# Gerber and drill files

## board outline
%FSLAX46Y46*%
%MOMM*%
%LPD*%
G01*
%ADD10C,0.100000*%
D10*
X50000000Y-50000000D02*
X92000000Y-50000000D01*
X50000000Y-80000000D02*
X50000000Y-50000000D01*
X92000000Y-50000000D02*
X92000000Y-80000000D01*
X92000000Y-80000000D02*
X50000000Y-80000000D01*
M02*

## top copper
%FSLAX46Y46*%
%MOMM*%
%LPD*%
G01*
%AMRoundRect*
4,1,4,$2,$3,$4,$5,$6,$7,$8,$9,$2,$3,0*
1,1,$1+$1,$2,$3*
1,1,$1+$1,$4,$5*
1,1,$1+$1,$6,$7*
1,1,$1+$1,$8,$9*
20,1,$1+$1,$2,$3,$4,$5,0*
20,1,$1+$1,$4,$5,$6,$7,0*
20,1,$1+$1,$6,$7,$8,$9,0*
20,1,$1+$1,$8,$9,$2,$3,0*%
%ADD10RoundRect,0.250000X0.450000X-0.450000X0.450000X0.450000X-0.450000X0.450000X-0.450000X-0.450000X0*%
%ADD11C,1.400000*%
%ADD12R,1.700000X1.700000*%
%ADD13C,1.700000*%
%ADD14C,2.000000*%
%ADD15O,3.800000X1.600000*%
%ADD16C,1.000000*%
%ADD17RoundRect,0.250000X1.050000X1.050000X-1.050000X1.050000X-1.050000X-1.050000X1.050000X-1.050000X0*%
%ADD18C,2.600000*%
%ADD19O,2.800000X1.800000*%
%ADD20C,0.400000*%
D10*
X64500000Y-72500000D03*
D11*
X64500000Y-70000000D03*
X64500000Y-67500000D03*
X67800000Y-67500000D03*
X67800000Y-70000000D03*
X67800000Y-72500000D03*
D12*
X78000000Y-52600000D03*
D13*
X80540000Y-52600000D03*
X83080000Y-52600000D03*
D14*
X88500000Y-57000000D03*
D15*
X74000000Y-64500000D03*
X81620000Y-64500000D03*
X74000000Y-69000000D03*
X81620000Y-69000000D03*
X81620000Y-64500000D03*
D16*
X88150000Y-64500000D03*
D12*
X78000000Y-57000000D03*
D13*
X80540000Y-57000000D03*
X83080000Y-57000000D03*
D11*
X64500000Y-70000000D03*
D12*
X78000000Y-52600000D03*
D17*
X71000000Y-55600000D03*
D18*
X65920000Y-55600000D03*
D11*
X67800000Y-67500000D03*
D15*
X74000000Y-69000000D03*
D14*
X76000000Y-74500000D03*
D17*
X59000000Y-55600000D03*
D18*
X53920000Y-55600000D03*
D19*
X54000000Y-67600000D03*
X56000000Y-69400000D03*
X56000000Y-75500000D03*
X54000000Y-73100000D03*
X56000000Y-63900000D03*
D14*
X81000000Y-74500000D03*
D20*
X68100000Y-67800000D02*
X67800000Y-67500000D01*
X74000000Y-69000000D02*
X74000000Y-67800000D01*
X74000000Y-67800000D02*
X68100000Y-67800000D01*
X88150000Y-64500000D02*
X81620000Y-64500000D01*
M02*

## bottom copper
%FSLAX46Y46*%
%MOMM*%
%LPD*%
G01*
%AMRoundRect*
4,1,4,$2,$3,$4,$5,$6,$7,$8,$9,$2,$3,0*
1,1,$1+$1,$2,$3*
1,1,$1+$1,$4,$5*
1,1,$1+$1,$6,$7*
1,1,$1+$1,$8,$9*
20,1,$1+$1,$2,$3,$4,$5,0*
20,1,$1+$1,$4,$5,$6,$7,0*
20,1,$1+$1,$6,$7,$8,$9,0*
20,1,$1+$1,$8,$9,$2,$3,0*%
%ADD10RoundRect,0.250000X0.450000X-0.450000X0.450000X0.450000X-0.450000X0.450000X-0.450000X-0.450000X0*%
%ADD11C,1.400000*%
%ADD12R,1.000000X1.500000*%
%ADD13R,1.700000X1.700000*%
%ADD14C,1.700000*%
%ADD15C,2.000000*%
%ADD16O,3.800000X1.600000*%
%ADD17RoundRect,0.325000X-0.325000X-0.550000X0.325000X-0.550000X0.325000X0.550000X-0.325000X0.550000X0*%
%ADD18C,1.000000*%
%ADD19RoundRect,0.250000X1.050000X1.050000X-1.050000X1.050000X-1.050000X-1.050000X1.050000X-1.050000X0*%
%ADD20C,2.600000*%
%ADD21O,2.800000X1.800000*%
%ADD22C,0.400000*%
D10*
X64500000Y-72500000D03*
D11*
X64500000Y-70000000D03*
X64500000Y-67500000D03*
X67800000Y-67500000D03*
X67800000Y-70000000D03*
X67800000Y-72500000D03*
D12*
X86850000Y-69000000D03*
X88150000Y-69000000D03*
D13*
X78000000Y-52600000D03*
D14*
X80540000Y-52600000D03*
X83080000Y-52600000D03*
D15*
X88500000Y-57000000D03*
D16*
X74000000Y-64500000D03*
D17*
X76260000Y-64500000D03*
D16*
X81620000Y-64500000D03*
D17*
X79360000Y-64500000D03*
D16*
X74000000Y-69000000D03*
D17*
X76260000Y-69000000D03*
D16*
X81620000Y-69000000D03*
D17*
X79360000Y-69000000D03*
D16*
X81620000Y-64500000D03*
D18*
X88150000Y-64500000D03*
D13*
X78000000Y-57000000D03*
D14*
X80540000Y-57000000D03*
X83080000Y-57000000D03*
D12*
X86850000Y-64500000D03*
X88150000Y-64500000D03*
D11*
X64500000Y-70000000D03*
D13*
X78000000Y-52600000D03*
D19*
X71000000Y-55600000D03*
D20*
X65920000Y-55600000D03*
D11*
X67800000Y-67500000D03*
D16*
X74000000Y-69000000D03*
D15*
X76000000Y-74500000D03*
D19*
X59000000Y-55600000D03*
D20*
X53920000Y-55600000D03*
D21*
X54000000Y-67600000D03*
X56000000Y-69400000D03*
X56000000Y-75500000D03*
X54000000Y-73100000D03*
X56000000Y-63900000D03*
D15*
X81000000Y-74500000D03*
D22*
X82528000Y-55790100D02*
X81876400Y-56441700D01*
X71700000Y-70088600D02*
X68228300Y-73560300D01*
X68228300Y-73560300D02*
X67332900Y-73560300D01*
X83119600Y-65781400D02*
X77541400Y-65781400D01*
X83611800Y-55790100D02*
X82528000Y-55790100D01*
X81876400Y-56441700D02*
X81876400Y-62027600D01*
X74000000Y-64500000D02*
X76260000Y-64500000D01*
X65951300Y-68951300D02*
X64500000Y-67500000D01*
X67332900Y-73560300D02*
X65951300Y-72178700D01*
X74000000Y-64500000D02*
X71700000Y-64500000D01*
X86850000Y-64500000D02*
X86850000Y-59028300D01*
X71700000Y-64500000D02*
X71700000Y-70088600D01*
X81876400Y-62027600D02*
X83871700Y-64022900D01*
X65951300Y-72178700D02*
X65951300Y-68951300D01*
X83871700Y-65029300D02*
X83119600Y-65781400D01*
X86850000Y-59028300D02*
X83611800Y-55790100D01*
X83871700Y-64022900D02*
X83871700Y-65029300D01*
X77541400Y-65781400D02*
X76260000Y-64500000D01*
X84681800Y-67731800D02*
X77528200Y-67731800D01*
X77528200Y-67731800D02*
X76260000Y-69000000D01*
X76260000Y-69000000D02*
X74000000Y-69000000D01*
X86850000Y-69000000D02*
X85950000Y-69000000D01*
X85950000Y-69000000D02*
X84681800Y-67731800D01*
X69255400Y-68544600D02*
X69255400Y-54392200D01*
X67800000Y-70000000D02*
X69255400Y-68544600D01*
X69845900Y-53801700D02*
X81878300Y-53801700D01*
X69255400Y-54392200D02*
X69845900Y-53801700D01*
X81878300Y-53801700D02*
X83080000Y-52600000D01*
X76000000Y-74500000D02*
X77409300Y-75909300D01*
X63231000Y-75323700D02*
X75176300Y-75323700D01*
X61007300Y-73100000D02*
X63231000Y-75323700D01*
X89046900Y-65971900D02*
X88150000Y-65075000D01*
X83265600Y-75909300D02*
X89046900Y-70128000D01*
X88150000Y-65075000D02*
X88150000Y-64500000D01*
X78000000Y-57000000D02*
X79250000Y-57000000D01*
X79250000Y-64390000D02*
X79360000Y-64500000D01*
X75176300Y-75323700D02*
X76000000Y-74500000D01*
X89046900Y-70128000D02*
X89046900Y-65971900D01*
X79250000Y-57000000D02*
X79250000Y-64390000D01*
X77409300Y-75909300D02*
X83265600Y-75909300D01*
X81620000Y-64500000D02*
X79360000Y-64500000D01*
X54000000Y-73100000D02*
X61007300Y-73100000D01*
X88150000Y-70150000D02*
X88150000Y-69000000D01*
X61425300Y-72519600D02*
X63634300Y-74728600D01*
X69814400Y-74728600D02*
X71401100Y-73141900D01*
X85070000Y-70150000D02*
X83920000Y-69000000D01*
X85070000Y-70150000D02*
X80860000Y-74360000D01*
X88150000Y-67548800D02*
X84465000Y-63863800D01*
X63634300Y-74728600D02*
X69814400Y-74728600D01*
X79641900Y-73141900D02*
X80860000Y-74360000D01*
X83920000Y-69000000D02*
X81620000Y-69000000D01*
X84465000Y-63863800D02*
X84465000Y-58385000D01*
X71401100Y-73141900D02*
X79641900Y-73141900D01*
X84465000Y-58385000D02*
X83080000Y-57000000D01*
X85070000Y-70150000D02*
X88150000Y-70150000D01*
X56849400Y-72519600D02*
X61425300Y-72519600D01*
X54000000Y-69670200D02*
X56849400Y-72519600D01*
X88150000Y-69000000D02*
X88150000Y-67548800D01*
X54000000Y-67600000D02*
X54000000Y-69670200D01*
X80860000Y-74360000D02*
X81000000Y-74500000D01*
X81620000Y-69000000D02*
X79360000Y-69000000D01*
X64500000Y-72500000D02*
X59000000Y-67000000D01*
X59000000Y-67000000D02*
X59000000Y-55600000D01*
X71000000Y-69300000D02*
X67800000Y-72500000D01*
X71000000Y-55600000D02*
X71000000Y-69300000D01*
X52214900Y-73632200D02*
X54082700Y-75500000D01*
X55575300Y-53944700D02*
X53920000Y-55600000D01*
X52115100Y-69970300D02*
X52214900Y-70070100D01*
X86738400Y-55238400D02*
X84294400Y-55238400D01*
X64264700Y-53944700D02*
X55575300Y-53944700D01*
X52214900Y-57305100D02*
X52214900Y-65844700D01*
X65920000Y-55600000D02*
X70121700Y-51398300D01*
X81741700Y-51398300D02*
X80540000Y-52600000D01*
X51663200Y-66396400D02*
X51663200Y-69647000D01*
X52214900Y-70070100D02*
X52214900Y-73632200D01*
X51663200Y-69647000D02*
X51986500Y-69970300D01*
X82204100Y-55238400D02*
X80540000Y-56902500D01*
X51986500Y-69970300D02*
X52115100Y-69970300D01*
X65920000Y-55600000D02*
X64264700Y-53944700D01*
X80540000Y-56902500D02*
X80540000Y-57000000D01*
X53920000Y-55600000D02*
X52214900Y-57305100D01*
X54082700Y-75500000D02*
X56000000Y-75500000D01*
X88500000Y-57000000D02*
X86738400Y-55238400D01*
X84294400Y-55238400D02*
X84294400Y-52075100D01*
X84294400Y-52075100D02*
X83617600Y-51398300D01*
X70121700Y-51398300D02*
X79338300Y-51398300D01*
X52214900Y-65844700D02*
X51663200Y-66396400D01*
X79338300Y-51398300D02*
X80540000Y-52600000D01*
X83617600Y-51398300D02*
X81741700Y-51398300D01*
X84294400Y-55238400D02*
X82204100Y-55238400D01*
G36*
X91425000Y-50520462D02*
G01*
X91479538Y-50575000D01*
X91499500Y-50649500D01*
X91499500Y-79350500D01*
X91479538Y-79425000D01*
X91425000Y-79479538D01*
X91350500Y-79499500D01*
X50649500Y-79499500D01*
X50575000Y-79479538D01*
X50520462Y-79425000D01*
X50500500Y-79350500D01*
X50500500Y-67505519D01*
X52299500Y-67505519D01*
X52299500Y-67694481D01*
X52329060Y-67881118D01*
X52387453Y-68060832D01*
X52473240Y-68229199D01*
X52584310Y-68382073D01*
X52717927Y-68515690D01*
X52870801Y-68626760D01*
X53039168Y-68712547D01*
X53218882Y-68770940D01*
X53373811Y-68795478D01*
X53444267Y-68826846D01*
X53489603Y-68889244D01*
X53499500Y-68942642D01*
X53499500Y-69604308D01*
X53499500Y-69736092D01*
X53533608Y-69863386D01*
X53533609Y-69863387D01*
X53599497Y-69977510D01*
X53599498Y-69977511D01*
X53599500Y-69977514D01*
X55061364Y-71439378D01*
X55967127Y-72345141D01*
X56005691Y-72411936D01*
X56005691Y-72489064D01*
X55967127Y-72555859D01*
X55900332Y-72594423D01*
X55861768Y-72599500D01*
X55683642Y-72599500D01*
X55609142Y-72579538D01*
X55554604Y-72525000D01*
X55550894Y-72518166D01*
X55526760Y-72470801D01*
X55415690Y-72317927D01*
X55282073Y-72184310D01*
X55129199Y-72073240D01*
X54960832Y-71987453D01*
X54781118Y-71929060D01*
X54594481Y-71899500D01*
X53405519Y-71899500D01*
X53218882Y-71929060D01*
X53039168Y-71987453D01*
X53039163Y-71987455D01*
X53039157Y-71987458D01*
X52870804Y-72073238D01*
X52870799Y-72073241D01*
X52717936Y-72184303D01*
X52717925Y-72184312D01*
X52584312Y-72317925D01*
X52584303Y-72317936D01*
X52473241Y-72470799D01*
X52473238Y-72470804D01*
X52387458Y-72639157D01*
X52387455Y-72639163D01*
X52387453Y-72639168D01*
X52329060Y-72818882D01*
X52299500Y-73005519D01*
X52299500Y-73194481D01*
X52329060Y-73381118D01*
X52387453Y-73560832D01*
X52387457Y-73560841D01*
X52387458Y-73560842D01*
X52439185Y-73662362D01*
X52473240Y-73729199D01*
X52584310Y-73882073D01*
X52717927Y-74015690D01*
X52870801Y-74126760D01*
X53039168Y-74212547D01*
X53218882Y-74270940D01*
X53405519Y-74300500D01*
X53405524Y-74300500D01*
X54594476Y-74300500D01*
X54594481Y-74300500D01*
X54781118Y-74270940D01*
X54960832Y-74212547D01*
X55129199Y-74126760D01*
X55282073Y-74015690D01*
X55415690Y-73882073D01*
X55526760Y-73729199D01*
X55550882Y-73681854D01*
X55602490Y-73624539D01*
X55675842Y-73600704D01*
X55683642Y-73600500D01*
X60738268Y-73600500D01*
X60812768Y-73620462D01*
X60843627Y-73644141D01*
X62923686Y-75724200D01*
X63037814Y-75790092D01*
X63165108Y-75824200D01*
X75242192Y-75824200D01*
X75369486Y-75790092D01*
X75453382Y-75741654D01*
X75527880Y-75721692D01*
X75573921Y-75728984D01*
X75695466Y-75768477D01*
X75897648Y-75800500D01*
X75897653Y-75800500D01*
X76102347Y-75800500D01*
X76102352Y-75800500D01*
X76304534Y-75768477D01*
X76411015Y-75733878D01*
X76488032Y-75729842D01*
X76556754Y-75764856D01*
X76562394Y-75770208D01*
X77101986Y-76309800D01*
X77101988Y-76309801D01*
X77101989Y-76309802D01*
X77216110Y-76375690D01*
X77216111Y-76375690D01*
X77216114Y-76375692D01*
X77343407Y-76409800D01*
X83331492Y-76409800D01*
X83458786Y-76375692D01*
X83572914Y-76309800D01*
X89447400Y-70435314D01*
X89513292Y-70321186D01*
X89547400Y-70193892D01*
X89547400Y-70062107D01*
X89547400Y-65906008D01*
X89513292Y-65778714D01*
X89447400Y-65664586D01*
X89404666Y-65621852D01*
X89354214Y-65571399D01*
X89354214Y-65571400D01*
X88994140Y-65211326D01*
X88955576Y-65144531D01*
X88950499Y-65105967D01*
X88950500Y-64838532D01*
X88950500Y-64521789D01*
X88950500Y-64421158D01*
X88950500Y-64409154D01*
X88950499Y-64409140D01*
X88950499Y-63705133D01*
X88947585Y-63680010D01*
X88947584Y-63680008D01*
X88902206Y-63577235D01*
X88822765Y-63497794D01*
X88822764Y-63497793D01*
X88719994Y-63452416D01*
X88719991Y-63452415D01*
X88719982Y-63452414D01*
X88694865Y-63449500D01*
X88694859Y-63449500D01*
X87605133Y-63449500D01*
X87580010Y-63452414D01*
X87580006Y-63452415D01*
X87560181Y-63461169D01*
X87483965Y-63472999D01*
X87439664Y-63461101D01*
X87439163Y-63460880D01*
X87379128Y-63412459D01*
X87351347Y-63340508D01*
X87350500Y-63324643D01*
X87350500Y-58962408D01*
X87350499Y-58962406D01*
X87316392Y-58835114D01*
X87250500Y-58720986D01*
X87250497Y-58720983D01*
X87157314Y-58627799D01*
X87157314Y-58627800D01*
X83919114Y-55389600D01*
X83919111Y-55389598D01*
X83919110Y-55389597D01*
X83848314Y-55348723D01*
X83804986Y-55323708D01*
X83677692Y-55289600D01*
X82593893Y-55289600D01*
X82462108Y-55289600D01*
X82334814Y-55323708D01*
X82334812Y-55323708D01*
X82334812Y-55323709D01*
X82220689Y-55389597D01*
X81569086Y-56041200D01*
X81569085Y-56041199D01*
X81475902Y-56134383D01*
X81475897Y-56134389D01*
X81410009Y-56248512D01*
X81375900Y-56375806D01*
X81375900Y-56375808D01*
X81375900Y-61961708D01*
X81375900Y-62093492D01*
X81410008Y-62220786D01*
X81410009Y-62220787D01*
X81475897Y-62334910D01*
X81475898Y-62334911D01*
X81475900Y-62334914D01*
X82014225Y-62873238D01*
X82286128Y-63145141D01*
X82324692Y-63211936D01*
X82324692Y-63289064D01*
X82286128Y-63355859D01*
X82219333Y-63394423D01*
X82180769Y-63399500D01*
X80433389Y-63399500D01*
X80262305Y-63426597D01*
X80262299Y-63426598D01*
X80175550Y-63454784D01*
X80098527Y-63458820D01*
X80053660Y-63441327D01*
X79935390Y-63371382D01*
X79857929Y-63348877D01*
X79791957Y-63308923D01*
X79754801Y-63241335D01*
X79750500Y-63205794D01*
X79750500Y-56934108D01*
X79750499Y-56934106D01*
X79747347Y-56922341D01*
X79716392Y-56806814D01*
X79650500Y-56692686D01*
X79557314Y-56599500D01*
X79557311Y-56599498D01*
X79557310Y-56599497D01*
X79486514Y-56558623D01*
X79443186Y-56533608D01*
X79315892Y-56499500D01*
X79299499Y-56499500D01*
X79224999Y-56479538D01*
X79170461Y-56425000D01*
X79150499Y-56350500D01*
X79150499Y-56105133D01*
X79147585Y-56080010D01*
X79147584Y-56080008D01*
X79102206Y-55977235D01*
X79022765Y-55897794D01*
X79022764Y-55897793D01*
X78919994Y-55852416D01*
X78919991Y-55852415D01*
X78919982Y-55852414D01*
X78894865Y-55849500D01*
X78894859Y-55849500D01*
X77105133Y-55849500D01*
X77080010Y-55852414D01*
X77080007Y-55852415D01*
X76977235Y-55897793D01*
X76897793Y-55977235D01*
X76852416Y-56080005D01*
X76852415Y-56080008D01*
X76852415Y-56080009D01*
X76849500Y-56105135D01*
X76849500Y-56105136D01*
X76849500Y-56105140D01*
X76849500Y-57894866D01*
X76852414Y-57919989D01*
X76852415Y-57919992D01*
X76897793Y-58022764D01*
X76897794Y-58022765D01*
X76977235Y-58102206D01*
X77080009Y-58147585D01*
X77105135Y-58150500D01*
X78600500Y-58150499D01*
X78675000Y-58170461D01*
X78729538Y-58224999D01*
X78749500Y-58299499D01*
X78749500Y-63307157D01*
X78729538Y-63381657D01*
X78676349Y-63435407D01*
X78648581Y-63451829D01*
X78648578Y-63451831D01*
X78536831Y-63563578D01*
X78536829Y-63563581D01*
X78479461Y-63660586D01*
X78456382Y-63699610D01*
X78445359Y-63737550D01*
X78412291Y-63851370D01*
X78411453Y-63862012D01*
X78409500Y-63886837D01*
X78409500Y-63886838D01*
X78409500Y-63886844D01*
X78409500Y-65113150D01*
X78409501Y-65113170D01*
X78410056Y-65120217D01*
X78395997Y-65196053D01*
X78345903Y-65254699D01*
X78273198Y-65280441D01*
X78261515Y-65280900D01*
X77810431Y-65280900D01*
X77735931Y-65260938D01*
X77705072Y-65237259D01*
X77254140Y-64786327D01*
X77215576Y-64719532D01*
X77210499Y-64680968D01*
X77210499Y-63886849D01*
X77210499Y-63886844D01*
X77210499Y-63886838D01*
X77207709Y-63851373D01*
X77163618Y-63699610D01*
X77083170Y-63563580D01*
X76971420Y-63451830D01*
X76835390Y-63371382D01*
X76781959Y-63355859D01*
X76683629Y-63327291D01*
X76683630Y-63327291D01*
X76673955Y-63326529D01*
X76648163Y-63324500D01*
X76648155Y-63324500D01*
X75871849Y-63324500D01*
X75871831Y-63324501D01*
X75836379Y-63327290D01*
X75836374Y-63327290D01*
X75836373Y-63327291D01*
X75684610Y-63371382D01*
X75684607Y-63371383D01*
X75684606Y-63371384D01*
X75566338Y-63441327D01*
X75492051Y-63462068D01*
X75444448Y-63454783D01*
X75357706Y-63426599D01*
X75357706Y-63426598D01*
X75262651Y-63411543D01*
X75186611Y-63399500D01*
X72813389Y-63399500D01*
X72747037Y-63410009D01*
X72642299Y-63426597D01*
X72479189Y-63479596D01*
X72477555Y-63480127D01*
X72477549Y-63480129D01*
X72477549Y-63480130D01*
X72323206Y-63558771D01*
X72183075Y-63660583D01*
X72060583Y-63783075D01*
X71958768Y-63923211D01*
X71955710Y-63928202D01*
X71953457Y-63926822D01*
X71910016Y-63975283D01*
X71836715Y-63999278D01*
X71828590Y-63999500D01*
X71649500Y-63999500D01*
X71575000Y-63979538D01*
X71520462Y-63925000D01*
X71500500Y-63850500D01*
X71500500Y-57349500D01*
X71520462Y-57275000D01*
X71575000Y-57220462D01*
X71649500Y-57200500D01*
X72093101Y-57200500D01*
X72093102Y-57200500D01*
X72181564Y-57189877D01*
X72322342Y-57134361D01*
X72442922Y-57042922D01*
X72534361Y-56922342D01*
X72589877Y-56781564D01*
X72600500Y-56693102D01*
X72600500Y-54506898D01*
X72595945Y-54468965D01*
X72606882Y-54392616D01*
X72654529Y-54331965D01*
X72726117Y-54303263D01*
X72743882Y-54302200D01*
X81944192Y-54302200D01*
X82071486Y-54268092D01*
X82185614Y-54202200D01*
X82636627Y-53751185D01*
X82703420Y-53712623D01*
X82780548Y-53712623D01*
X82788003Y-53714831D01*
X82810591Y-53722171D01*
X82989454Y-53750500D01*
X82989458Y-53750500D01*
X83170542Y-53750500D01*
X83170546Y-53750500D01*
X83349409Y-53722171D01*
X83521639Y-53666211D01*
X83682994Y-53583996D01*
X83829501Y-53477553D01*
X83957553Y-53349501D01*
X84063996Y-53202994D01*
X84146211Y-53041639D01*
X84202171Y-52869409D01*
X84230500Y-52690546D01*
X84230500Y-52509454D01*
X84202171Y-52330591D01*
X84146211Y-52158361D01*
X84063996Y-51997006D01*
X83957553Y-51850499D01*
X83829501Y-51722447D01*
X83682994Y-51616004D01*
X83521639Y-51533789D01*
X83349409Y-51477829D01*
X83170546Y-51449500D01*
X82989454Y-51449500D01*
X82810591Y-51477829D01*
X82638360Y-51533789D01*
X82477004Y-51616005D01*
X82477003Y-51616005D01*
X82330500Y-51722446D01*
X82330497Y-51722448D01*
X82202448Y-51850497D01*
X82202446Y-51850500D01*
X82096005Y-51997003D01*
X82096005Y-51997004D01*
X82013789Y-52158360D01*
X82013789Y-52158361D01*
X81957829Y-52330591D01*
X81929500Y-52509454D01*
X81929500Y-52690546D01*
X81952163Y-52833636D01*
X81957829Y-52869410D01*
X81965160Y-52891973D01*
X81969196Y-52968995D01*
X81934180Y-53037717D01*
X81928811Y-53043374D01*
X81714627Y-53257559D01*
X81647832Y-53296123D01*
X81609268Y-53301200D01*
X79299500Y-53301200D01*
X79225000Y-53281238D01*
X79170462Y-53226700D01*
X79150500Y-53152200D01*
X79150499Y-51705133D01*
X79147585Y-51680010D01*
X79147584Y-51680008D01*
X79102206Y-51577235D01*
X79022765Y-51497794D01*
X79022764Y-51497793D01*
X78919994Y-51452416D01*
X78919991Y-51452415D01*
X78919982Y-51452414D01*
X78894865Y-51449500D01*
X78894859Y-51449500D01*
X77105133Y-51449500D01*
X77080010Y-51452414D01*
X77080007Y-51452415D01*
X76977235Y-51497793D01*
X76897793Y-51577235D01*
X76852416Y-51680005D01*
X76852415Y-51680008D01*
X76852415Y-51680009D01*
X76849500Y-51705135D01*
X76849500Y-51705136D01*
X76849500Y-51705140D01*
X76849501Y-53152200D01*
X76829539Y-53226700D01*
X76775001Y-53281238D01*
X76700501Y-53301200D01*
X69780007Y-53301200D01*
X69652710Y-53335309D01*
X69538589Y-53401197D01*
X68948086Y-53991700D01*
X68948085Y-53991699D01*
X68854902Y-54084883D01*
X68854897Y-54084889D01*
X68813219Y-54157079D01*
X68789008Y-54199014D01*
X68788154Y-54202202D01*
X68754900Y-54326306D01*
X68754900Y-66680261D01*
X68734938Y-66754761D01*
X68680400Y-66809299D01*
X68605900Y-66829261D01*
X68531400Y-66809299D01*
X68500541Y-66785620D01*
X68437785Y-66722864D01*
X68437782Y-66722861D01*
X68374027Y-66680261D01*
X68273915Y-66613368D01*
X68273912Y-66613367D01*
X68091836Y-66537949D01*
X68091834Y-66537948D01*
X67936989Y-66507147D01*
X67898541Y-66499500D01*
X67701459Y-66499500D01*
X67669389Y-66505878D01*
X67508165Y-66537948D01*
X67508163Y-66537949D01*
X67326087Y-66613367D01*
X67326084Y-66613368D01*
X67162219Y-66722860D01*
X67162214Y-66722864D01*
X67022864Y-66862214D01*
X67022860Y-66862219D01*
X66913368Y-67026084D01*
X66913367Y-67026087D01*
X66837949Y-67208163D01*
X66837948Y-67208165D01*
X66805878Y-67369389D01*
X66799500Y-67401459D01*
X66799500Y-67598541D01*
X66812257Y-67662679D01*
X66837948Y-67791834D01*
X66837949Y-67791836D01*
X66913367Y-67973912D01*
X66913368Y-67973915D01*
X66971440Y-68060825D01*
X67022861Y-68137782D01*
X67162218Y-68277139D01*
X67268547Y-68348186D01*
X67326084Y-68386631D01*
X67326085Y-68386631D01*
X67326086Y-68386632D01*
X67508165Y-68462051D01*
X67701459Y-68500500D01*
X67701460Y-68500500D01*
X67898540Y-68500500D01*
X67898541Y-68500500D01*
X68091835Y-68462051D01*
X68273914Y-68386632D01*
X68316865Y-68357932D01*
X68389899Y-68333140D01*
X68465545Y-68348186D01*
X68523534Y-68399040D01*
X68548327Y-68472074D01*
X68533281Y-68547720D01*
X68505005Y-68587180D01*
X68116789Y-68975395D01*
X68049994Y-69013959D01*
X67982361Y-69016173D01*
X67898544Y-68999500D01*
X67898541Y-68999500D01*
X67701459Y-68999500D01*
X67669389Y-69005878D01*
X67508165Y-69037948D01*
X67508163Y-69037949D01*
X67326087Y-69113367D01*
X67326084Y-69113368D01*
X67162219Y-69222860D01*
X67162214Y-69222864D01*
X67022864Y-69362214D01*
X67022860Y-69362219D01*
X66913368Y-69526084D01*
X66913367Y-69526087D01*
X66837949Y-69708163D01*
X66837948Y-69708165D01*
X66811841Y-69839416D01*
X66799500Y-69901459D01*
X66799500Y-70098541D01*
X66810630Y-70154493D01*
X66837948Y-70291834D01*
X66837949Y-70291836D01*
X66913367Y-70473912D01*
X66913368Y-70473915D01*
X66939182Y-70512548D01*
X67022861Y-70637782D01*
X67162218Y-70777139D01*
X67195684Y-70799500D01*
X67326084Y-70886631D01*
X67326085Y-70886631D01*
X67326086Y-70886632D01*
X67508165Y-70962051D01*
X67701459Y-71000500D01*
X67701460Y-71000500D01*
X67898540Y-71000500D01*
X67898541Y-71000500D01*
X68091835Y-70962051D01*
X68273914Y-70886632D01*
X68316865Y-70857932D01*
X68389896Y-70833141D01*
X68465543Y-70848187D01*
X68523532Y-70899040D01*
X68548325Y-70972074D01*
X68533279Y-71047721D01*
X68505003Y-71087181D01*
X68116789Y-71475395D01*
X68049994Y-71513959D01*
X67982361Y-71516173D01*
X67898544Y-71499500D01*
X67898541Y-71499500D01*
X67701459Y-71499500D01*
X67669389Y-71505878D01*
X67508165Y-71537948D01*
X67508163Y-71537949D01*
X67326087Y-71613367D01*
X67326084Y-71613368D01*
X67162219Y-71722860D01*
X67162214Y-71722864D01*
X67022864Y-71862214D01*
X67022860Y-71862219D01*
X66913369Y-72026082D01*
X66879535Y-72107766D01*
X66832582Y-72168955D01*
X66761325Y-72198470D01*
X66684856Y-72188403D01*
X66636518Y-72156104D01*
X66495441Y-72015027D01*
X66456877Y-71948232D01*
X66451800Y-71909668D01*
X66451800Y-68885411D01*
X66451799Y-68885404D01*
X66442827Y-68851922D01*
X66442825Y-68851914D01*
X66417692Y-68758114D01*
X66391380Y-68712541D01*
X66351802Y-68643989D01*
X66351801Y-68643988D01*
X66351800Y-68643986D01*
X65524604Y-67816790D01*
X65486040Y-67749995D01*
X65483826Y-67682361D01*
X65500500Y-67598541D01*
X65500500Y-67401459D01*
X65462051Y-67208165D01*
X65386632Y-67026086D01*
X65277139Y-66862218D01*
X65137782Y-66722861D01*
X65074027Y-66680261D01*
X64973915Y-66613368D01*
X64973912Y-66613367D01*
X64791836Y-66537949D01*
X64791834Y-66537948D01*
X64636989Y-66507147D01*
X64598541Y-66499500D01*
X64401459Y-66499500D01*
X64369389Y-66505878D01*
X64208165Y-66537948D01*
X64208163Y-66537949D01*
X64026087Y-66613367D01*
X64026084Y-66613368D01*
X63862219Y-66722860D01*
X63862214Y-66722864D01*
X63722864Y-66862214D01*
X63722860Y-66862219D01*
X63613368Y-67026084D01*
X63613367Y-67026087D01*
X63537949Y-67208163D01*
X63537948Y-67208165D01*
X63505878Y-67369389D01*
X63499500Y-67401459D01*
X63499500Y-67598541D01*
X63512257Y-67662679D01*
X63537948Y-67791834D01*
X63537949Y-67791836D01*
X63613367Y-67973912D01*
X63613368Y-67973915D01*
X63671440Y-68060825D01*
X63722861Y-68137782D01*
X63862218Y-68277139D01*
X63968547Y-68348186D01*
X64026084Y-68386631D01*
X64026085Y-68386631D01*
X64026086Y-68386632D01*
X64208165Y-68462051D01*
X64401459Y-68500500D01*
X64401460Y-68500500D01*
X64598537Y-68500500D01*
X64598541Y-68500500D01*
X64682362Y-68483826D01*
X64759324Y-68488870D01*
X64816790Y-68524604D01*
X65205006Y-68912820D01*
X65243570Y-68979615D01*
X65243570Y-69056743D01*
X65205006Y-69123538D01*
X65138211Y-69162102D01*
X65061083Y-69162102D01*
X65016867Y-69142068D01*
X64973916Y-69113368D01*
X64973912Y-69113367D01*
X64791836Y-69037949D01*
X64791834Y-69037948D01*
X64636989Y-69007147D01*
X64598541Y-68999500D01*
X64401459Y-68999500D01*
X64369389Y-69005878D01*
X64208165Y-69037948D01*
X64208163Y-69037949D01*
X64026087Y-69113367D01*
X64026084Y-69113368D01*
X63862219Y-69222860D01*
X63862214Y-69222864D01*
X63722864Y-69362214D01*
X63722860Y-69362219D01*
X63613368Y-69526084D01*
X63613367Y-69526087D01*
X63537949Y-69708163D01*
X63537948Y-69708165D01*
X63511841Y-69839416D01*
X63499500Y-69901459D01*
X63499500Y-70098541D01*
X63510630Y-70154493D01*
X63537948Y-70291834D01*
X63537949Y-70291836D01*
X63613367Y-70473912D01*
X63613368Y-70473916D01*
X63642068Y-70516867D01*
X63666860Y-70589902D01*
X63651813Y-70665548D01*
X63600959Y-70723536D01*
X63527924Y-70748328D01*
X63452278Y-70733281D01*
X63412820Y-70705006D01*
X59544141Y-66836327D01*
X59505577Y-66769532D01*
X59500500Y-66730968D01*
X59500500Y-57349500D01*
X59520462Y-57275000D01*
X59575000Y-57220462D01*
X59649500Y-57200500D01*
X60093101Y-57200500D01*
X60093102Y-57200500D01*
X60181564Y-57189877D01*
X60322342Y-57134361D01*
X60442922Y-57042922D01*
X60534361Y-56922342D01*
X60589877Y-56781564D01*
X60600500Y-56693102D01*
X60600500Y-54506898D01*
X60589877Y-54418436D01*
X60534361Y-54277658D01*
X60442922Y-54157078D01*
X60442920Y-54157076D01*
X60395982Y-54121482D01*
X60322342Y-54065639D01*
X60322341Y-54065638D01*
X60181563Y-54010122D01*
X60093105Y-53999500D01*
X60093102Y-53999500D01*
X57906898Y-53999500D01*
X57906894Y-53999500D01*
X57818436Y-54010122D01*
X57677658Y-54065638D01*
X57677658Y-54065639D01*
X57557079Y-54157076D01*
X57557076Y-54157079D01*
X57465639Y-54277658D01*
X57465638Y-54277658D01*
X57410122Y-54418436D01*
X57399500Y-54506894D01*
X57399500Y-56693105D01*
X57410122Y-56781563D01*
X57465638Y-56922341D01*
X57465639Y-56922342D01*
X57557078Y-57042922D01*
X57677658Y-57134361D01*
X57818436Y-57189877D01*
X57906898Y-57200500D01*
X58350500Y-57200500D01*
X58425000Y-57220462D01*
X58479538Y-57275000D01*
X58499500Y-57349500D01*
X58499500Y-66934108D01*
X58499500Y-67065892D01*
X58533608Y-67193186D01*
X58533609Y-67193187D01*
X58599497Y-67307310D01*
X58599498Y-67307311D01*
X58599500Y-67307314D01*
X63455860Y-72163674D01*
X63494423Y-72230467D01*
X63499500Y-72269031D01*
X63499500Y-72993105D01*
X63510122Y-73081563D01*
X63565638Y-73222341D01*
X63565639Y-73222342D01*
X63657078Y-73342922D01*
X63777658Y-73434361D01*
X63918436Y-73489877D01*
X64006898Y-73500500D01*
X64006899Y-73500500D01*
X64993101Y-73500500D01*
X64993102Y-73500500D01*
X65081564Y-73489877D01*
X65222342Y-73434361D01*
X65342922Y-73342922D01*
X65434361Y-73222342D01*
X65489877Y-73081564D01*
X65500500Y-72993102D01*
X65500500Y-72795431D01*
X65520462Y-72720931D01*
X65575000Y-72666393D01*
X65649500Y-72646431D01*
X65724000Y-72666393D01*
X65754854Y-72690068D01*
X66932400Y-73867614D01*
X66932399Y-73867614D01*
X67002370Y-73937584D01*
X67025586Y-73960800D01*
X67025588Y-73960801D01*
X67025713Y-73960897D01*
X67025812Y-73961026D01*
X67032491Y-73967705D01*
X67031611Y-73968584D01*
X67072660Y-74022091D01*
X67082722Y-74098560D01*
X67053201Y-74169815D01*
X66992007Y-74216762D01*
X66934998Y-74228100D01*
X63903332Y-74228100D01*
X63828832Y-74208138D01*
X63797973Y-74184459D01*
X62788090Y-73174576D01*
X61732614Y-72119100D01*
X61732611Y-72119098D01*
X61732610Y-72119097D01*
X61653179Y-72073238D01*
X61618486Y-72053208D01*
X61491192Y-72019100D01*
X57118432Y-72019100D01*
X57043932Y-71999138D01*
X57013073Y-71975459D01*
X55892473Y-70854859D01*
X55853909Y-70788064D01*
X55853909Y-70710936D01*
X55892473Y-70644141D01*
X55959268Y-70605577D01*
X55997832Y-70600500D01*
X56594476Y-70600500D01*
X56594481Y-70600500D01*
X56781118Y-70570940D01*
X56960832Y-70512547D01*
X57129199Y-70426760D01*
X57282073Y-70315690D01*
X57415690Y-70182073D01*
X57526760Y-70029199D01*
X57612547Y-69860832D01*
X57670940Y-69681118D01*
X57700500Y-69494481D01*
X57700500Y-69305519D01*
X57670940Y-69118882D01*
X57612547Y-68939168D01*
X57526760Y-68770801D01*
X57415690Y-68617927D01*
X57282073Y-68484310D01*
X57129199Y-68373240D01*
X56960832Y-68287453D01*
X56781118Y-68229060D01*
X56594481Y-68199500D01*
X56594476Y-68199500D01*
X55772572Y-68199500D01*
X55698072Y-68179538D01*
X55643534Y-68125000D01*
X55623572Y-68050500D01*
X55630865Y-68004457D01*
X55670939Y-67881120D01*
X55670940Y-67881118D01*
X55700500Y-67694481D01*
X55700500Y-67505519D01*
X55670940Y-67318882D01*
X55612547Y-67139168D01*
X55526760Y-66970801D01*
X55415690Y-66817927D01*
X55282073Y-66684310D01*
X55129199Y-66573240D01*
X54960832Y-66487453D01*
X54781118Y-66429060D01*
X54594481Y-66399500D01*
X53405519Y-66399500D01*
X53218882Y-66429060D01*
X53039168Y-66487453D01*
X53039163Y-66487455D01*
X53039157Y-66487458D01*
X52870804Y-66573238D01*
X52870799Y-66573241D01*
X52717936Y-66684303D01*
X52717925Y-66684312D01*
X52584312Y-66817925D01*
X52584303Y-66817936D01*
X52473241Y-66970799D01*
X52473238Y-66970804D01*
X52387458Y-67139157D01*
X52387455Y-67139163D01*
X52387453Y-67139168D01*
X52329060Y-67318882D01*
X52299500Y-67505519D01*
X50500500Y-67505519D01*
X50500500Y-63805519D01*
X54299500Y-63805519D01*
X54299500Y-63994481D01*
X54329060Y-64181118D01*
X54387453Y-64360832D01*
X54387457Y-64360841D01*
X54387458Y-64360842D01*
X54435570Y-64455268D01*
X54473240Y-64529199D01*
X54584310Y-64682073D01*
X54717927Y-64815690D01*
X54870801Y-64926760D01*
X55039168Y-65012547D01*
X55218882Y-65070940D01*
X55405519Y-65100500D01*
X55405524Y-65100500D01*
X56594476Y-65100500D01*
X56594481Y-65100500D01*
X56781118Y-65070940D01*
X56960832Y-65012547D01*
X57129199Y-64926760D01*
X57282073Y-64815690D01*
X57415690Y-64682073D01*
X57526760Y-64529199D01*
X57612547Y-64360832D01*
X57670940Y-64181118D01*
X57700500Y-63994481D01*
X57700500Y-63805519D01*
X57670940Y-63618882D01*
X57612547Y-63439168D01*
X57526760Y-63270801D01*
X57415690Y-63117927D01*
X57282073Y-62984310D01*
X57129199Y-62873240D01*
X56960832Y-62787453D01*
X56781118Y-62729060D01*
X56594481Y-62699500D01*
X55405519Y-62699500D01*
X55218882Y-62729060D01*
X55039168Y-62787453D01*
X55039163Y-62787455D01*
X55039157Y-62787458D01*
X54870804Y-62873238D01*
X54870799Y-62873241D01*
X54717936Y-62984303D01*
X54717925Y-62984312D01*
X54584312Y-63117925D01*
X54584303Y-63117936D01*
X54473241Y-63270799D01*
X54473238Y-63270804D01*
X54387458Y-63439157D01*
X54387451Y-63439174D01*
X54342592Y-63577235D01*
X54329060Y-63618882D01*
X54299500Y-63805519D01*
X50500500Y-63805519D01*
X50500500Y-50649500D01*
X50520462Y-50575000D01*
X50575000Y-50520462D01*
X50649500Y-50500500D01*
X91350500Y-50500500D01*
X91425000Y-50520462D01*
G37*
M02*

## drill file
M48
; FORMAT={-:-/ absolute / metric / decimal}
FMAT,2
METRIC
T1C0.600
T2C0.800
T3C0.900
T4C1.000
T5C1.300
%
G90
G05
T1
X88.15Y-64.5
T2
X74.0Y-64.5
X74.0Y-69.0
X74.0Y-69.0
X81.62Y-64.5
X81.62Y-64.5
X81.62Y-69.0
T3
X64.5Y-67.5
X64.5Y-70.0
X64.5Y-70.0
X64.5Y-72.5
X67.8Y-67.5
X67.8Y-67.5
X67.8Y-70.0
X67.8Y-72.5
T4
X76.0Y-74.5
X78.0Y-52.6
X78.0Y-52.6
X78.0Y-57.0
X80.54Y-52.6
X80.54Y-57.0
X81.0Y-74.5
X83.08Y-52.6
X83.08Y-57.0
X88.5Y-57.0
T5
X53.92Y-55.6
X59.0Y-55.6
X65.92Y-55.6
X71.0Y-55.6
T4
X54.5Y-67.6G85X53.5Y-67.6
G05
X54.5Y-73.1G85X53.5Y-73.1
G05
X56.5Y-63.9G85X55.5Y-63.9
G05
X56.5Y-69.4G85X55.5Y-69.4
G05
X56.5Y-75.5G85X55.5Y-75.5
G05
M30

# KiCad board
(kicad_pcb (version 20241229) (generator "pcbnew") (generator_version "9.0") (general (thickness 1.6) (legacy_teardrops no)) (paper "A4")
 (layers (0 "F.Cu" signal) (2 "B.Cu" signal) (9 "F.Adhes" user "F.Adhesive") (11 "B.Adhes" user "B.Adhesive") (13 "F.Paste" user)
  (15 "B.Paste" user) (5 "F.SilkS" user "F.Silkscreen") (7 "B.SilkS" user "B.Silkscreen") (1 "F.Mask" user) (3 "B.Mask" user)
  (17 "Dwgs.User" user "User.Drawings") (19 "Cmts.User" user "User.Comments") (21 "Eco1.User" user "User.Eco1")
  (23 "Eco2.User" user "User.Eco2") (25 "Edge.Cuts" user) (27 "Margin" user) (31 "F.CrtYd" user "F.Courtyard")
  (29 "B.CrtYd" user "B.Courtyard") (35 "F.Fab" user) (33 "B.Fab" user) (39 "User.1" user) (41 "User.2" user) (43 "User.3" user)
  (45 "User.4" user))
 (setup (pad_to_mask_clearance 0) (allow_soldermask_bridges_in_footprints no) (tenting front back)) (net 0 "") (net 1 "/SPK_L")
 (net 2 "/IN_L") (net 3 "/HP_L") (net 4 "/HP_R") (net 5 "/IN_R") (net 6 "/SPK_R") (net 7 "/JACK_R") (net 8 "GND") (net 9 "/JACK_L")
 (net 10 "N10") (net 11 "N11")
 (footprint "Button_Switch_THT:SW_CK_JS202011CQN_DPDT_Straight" (layer "F.Cu") (at 64.5 72.5 90)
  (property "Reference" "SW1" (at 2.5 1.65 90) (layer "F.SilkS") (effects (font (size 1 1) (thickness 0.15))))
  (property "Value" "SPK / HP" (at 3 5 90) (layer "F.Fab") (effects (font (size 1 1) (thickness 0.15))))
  (pad "1" thru_hole roundrect (at 0 0 90) (size 1.4 1.4) (drill 0.9) (layers "*.Cu" "*.Mask") (remove_unused_layers no)
   (roundrect_rratio 0.1785714286) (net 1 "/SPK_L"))
  (pad "2" thru_hole circle (at 2.5 0 90) (size 1.4 1.4) (drill 0.9) (layers "*.Cu" "*.Mask") (remove_unused_layers no) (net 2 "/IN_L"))
  (pad "3" thru_hole circle (at 5 0 90) (size 1.4 1.4) (drill 0.9) (layers "*.Cu" "*.Mask") (remove_unused_layers no) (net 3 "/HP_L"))
  (pad "4" thru_hole circle (at 5 3.3 90) (size 1.4 1.4) (drill 0.9) (layers "*.Cu" "*.Mask") (remove_unused_layers no) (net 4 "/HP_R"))
  (pad "5" thru_hole circle (at 2.5 3.3 90) (size 1.4 1.4) (drill 0.9) (layers "*.Cu" "*.Mask") (remove_unused_layers no) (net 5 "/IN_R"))
  (pad "6" thru_hole circle (at 0 3.3 90) (size 1.4 1.4) (drill 0.9) (layers "*.Cu" "*.Mask") (remove_unused_layers no) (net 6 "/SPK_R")))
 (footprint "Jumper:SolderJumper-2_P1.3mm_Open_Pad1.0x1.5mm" (layer "F.Cu") (at 87.5 69)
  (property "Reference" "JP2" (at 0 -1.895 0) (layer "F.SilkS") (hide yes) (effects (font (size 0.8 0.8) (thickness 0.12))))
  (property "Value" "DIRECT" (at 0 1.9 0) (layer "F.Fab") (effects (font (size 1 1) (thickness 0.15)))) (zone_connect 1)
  (pad "1" smd rect (at -0.65 0) (size 1 1.5) (layers "B.Cu" "B.Mask" "B.Paste") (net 4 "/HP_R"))
  (pad "2" smd rect (at 0.65 0) (size 1 1.5) (layers "B.Cu" "B.Mask" "B.Paste") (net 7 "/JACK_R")))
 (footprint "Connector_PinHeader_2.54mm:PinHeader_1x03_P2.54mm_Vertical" (layer "F.Cu") (at 78 52.6 90)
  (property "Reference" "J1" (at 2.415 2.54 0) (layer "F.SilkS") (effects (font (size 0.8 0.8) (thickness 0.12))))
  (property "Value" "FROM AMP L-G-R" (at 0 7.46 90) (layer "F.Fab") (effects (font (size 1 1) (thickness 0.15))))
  (pad "1" thru_hole rect (at 0 0 90) (size 1.7 1.7) (drill 1) (layers "*.Cu" "*.Mask") (remove_unused_layers no) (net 2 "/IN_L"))
  (pad "2" thru_hole circle (at 0 2.54 90) (size 1.7 1.7) (drill 1) (layers "*.Cu" "*.Mask") (remove_unused_layers no) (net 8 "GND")
   (zone_connect 2))
  (pad "3" thru_hole circle (at 0 5.08 90) (size 1.7 1.7) (drill 1) (layers "*.Cu" "*.Mask") (remove_unused_layers no) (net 5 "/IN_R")))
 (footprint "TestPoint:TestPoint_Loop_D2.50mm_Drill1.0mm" (layer "F.Cu") (at 88.5 57)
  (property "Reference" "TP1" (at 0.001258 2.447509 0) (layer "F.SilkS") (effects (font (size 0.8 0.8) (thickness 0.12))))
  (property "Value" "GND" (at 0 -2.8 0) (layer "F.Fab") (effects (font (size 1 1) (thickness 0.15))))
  (pad "1" thru_hole circle (at 0 0) (size 2 2) (drill 1) (layers "*.Cu" "*.Mask") (remove_unused_layers no) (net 8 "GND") (zone_connect 2)))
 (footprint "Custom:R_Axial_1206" (layer "F.Cu") (at 74 64.5)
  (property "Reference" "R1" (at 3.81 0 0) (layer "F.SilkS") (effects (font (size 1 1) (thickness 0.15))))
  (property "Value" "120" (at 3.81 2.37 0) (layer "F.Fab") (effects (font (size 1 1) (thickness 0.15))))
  (pad "1" thru_hole oval (at 0 0) (size 3.8 1.6) (drill 0.8) (layers "*.Cu" "*.Mask") (remove_unused_layers no) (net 3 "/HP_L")
   (thermal_bridge_angle 45))
  (pad "1S" smd roundrect (at 2.26 0) (size 1.3 1.75) (layers "B.Cu" "B.Mask" "B.Paste") (roundrect_rratio 0.25) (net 3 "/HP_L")
   (zone_connect 2) (thermal_bridge_angle 45))
  (pad "2" thru_hole oval (at 7.62 0) (size 3.8 1.6) (drill 0.8) (layers "*.Cu" "*.Mask") (remove_unused_layers no) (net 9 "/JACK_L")
   (thermal_bridge_angle 45))
  (pad "2S" smd roundrect (at 5.36 0) (size 1.3 1.75) (layers "B.Cu" "B.Mask" "B.Paste") (roundrect_rratio 0.25) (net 9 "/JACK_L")
   (zone_connect 2) (thermal_bridge_angle 45)))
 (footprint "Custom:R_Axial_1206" (layer "F.Cu") (at 74 69)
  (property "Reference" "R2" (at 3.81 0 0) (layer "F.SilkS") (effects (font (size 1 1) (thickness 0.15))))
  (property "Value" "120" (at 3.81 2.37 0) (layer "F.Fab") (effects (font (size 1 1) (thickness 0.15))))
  (pad "1" thru_hole oval (at 0 0) (size 3.8 1.6) (drill 0.8) (layers "*.Cu" "*.Mask") (remove_unused_layers no) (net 4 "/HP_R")
   (thermal_bridge_angle 45))
  (pad "1S" smd roundrect (at 2.26 0) (size 1.3 1.75) (layers "B.Cu" "B.Mask" "B.Paste") (roundrect_rratio 0.25) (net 4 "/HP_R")
   (zone_connect 2) (thermal_bridge_angle 45))
  (pad "2" thru_hole oval (at 7.62 0) (size 3.8 1.6) (drill 0.8) (layers "*.Cu" "*.Mask") (remove_unused_layers no) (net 7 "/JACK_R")
   (thermal_bridge_angle 45))
  (pad "2S" smd roundrect (at 5.36 0) (size 1.3 1.75) (layers "B.Cu" "B.Mask" "B.Paste") (roundrect_rratio 0.25) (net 7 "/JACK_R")
   (zone_connect 2) (thermal_bridge_angle 45)))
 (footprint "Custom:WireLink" (layer "F.Cu") (at 81.62 64.5)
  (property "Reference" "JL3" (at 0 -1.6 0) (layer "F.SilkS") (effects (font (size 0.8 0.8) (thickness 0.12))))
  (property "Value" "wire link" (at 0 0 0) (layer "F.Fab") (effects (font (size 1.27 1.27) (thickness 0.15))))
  (pad "1" thru_hole oval (at 0 0) (size 3.8 1.6) (drill 0.8) (layers "*.Cu" "*.Mask") (remove_unused_layers no) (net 9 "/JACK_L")
   (thermal_bridge_angle 45))
  (pad "2" thru_hole circle (at 6.53 0) (size 1 1) (drill 0.6) (layers "*.Cu" "*.Mask") (remove_unused_layers no) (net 9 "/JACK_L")))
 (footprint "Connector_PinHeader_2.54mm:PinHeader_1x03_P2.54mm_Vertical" (layer "F.Cu") (at 78 57 90)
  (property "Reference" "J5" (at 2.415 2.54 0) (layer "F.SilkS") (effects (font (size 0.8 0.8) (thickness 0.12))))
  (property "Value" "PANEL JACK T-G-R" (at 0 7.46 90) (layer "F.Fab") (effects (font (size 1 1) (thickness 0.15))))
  (pad "1" thru_hole rect (at 0 0 90) (size 1.7 1.7) (drill 1) (layers "*.Cu" "*.Mask") (remove_unused_layers no) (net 9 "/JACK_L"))
  (pad "2" thru_hole circle (at 0 2.54 90) (size 1.7 1.7) (drill 1) (layers "*.Cu" "*.Mask") (remove_unused_layers no) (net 8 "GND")
   (zone_connect 2))
  (pad "3" thru_hole circle (at 0 5.08 90) (size 1.7 1.7) (drill 1) (layers "*.Cu" "*.Mask") (remove_unused_layers no) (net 7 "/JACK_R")))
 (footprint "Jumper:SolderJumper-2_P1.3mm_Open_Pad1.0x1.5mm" (layer "F.Cu") (at 87.5 64.5)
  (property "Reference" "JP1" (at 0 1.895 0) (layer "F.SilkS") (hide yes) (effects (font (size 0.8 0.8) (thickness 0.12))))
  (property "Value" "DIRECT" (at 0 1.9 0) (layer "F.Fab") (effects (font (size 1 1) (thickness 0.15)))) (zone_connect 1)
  (pad "1" smd rect (at -0.65 0) (size 1 1.5) (layers "B.Cu" "B.Mask" "B.Paste") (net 3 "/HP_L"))
  (pad "2" smd rect (at 0.65 0) (size 1 1.5) (layers "B.Cu" "B.Mask" "B.Paste") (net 9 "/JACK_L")))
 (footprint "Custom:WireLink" (layer "F.Cu") (at 64.5 70)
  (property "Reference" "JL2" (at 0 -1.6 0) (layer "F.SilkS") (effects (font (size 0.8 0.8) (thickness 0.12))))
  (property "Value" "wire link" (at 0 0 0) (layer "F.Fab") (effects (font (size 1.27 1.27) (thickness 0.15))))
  (pad "1" thru_hole circle (at 0 0) (size 1.4 1.4) (drill 0.9) (layers "*.Cu" "*.Mask") (remove_unused_layers no) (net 2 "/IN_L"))
  (pad "2" thru_hole rect (at 13.5 -17.4) (size 1.7 1.7) (drill 1) (layers "*.Cu" "*.Mask") (remove_unused_layers no) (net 2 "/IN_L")
   (thermal_bridge_angle 45)))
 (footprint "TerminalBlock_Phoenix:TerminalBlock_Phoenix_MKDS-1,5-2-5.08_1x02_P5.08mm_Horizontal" (layer "F.Cu") (at 71 55.6 180)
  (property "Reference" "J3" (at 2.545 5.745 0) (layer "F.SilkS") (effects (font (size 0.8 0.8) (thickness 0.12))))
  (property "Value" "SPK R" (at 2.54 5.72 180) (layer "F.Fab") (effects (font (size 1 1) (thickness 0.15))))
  (pad "1" thru_hole roundrect (at 0 0 180) (size 2.6 2.6) (drill 1.3) (layers "*.Cu" "*.Mask") (remove_unused_layers no)
   (roundrect_rratio 0.096154) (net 6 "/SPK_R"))
  (pad "2" thru_hole circle (at 5.08 0 180) (size 2.6 2.6) (drill 1.3) (layers "*.Cu" "*.Mask") (remove_unused_layers no) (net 8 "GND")
   (zone_connect 2)))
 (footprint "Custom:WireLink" (layer "F.Cu") (at 67.8 67.5)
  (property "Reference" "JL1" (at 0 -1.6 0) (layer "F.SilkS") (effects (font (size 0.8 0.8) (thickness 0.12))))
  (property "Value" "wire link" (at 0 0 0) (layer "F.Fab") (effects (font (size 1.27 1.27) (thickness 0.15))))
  (pad "1" thru_hole circle (at 0 0) (size 1.4 1.4) (drill 0.9) (layers "*.Cu" "*.Mask") (remove_unused_layers no) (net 4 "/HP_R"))
  (pad "2" thru_hole oval (at 6.2 1.5) (size 3.8 1.6) (drill 0.8) (layers "*.Cu" "*.Mask") (remove_unused_layers no) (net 4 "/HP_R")
   (thermal_bridge_angle 45)))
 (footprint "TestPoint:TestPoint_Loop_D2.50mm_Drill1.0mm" (layer "F.Cu") (at 76 74.5)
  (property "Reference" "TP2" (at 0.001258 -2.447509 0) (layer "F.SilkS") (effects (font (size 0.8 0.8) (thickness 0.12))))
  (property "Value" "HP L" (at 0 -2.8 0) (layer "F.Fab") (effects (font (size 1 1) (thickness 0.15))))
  (pad "1" thru_hole circle (at 0 0) (size 2 2) (drill 1) (layers "*.Cu" "*.Mask") (remove_unused_layers no) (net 9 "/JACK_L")))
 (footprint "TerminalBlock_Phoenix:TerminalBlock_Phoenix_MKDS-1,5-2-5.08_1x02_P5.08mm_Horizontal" (layer "F.Cu") (at 59 55.6 180)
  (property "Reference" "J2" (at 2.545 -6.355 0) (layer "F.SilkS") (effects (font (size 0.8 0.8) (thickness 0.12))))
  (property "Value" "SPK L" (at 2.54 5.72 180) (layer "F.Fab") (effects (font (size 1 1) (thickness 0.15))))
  (pad "1" thru_hole roundrect (at 0 0 180) (size 2.6 2.6) (drill 1.3) (layers "*.Cu" "*.Mask") (remove_unused_layers no)
   (roundrect_rratio 0.096154) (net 1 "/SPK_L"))
  (pad "2" thru_hole circle (at 5.08 0 180) (size 2.6 2.6) (drill 1.3) (layers "*.Cu" "*.Mask") (remove_unused_layers no) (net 8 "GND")
   (zone_connect 2)))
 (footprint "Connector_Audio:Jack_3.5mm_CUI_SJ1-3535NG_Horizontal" (layer "F.Cu") (at 56 75.5 180)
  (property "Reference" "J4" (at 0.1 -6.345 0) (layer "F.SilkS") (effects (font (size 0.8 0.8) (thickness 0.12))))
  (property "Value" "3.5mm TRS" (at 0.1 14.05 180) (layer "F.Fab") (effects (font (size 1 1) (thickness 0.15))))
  (pad "R" thru_hole oval (at 2 7.9 180) (size 2.8 1.8) (drill oval 2 1) (layers "*.Cu" "*.Mask") (remove_unused_layers no)
   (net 7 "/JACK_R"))
  (pad "RN" thru_hole oval (at 0 6.1 180) (size 2.8 1.8) (drill oval 2 1) (layers "*.Cu" "*.Mask") (remove_unused_layers no) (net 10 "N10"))
  (pad "S" thru_hole oval (at 0 0 180) (size 2.8 1.8) (drill oval 2 1) (layers "*.Cu" "*.Mask") (remove_unused_layers no) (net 8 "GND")
   (zone_connect 2))
  (pad "T" thru_hole oval (at 2 2.4 180) (size 2.8 1.8) (drill oval 2 1) (layers "*.Cu" "*.Mask") (remove_unused_layers no)
   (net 9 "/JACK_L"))
  (pad "TN" thru_hole oval (at 0 11.6 180) (size 2.8 1.8) (drill oval 2 1) (layers "*.Cu" "*.Mask") (remove_unused_layers no) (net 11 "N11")))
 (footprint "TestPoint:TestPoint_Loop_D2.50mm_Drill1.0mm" (layer "F.Cu") (at 81 74.5)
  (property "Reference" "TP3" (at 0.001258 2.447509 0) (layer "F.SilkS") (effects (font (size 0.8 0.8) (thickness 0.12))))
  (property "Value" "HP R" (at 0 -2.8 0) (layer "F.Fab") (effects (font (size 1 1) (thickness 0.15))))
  (pad "1" thru_hole circle (at 0 0) (size 2 2) (drill 1) (layers "*.Cu" "*.Mask") (remove_unused_layers no) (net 7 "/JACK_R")))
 (gr_line (start 50 50) (end 92 50) (stroke (width 0.1) (type default)) (layer "Edge.Cuts"))
 (gr_line (start 50 80) (end 50 50) (stroke (width 0.1) (type default)) (layer "Edge.Cuts"))
 (gr_line (start 92 50) (end 92 80) (stroke (width 0.1) (type default)) (layer "Edge.Cuts"))
 (gr_line (start 92 80) (end 50 80) (stroke (width 0.1) (type default)) (layer "Edge.Cuts"))
 (segment (start 82.528 55.7901) (end 81.8764 56.4417) (width 0.4) (layer "B.Cu") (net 3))
 (segment (start 71.7 70.0886) (end 68.2283 73.5603) (width 0.4) (layer "B.Cu") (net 3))
 (segment (start 68.2283 73.5603) (end 67.3329 73.5603) (width 0.4) (layer "B.Cu") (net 3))
 (segment (start 83.1196 65.7814) (end 77.5414 65.7814) (width 0.4) (layer "B.Cu") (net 3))
 (segment (start 83.6118 55.7901) (end 82.528 55.7901) (width 0.4) (layer "B.Cu") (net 3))
 (segment (start 81.8764 56.4417) (end 81.8764 62.0276) (width 0.4) (layer "B.Cu") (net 3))
 (segment (start 74 64.5) (end 76.26 64.5) (width 0.4) (layer "B.Cu") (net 3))
 (segment (start 65.9513 68.9513) (end 64.5 67.5) (width 0.4) (layer "B.Cu") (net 3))
 (segment (start 67.3329 73.5603) (end 65.9513 72.1787) (width 0.4) (layer "B.Cu") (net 3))
 (segment (start 74 64.5) (end 71.7 64.5) (width 0.4) (layer "B.Cu") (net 3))
 (segment (start 86.85 64.5) (end 86.85 59.0283) (width 0.4) (layer "B.Cu") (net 3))
 (segment (start 71.7 64.5) (end 71.7 70.0886) (width 0.4) (layer "B.Cu") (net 3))
 (segment (start 81.8764 62.0276) (end 83.8717 64.0229) (width 0.4) (layer "B.Cu") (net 3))
 (segment (start 65.9513 72.1787) (end 65.9513 68.9513) (width 0.4) (layer "B.Cu") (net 3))
 (segment (start 83.8717 65.0293) (end 83.1196 65.7814) (width 0.4) (layer "B.Cu") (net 3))
 (segment (start 86.85 59.0283) (end 83.6118 55.7901) (width 0.4) (layer "B.Cu") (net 3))
 (segment (start 83.8717 64.0229) (end 83.8717 65.0293) (width 0.4) (layer "B.Cu") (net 3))
 (segment (start 77.5414 65.7814) (end 76.26 64.5) (width 0.4) (layer "B.Cu") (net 3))
 (segment (start 68.1 67.8) (end 67.8 67.5) (width 0.4) (layer "F.Cu") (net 4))
 (segment (start 74 69) (end 74 67.8) (width 0.4) (layer "F.Cu") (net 4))
 (segment (start 74 67.8) (end 68.1 67.8) (width 0.4) (layer "F.Cu") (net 4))
 (segment (start 84.6818 67.7318) (end 77.5282 67.7318) (width 0.4) (layer "B.Cu") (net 4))
 (segment (start 77.5282 67.7318) (end 76.26 69) (width 0.4) (layer "B.Cu") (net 4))
 (segment (start 76.26 69) (end 74 69) (width 0.4) (layer "B.Cu") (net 4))
 (segment (start 86.85 69) (end 85.95 69) (width 0.4) (layer "B.Cu") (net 4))
 (segment (start 85.95 69) (end 84.6818 67.7318) (width 0.4) (layer "B.Cu") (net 4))
 (segment (start 69.2554 68.5446) (end 69.2554 54.3922) (width 0.4) (layer "B.Cu") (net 5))
 (segment (start 67.8 70) (end 69.2554 68.5446) (width 0.4) (layer "B.Cu") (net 5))
 (segment (start 69.8459 53.8017) (end 81.8783 53.8017) (width 0.4) (layer "B.Cu") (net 5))
 (segment (start 69.2554 54.3922) (end 69.8459 53.8017) (width 0.4) (layer "B.Cu") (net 5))
 (segment (start 81.8783 53.8017) (end 83.08 52.6) (width 0.4) (layer "B.Cu") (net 5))
 (segment (start 88.15 64.5) (end 81.62 64.5) (width 0.4) (layer "F.Cu") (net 9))
 (segment (start 76 74.5) (end 77.4093 75.9093) (width 0.4) (layer "B.Cu") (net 9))
 (segment (start 63.231 75.3237) (end 75.1763 75.3237) (width 0.4) (layer "B.Cu") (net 9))
 (segment (start 61.0073 73.1) (end 63.231 75.3237) (width 0.4) (layer "B.Cu") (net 9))
 (segment (start 89.0469 65.9719) (end 88.15 65.075) (width 0.4) (layer "B.Cu") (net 9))
 (segment (start 83.2656 75.9093) (end 89.0469 70.128) (width 0.4) (layer "B.Cu") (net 9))
 (segment (start 88.15 65.075) (end 88.15 64.5) (width 0.4) (layer "B.Cu") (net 9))
 (segment (start 78 57) (end 79.25 57) (width 0.4) (layer "B.Cu") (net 9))
 (segment (start 79.25 64.39) (end 79.36 64.5) (width 0.4) (layer "B.Cu") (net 9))
 (segment (start 75.1763 75.3237) (end 76 74.5) (width 0.4) (layer "B.Cu") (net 9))
 (segment (start 89.0469 70.128) (end 89.0469 65.9719) (width 0.4) (layer "B.Cu") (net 9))
 (segment (start 79.25 57) (end 79.25 64.39) (width 0.4) (layer "B.Cu") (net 9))
 (segment (start 77.4093 75.9093) (end 83.2656 75.9093) (width 0.4) (layer "B.Cu") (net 9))
 (segment (start 81.62 64.5) (end 79.36 64.5) (width 0.4) (layer "B.Cu") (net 9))
 (segment (start 54 73.1) (end 61.0073 73.1) (width 0.4) (layer "B.Cu") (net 9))
 (segment (start 88.15 70.15) (end 88.15 69) (width 0.4) (layer "B.Cu") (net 7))
 (segment (start 61.4253 72.5196) (end 63.6343 74.7286) (width 0.4) (layer "B.Cu") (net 7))
 (segment (start 69.8144 74.7286) (end 71.4011 73.1419) (width 0.4) (layer "B.Cu") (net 7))
 (segment (start 85.07 70.15) (end 83.92 69) (width 0.4) (layer "B.Cu") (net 7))
 (segment (start 85.07 70.15) (end 80.86 74.36) (width 0.4) (layer "B.Cu") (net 7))
 (segment (start 88.15 67.5488) (end 84.465 63.8638) (width 0.4) (layer "B.Cu") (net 7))
 (segment (start 63.6343 74.7286) (end 69.8144 74.7286) (width 0.4) (layer "B.Cu") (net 7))
 (segment (start 79.6419 73.1419) (end 80.86 74.36) (width 0.4) (layer "B.Cu") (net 7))
 (segment (start 83.92 69) (end 81.62 69) (width 0.4) (layer "B.Cu") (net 7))
 (segment (start 84.465 63.8638) (end 84.465 58.385) (width 0.4) (layer "B.Cu") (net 7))
 (segment (start 71.4011 73.1419) (end 79.6419 73.1419) (width 0.4) (layer "B.Cu") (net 7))
 (segment (start 84.465 58.385) (end 83.08 57) (width 0.4) (layer "B.Cu") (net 7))
 (segment (start 85.07 70.15) (end 88.15 70.15) (width 0.4) (layer "B.Cu") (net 7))
 (segment (start 56.8494 72.5196) (end 61.4253 72.5196) (width 0.4) (layer "B.Cu") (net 7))
 (segment (start 54 69.6702) (end 56.8494 72.5196) (width 0.4) (layer "B.Cu") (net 7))
 (segment (start 88.15 69) (end 88.15 67.5488) (width 0.4) (layer "B.Cu") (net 7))
 (segment (start 54 67.6) (end 54 69.6702) (width 0.4) (layer "B.Cu") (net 7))
 (segment (start 80.86 74.36) (end 81 74.5) (width 0.4) (layer "B.Cu") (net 7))
 (segment (start 81.62 69) (end 79.36 69) (width 0.4) (layer "B.Cu") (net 7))
 (segment (start 64.5 72.5) (end 59 67) (width 0.4) (layer "B.Cu") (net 1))
 (segment (start 59 67) (end 59 55.6) (width 0.4) (layer "B.Cu") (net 1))
 (segment (start 71 69.3) (end 67.8 72.5) (width 0.4) (layer "B.Cu") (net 6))
 (segment (start 71 55.6) (end 71 69.3) (width 0.4) (layer "B.Cu") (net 6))
 (segment (start 52.2149 73.6322) (end 54.0827 75.5) (width 0.4) (layer "B.Cu") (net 8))
 (segment (start 55.5753 53.9447) (end 53.92 55.6) (width 0.4) (layer "B.Cu") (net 8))
 (segment (start 52.1151 69.9703) (end 52.2149 70.0701) (width 0.4) (layer "B.Cu") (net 8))
 (segment (start 86.7384 55.2384) (end 84.2944 55.2384) (width 0.4) (layer "B.Cu") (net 8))
 (segment (start 64.2647 53.9447) (end 55.5753 53.9447) (width 0.4) (layer "B.Cu") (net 8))
 (segment (start 52.2149 57.3051) (end 52.2149 65.8447) (width 0.4) (layer "B.Cu") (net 8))
 (segment (start 65.92 55.6) (end 70.1217 51.3983) (width 0.4) (layer "B.Cu") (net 8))
 (segment (start 81.7417 51.3983) (end 80.54 52.6) (width 0.4) (layer "B.Cu") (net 8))
 (segment (start 51.6632 66.3964) (end 51.6632 69.647) (width 0.4) (layer "B.Cu") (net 8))
 (segment (start 52.2149 70.0701) (end 52.2149 73.6322) (width 0.4) (layer "B.Cu") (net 8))
 (segment (start 51.6632 69.647) (end 51.9865 69.9703) (width 0.4) (layer "B.Cu") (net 8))
 (segment (start 82.2041 55.2384) (end 80.54 56.9025) (width 0.4) (layer "B.Cu") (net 8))
 (segment (start 51.9865 69.9703) (end 52.1151 69.9703) (width 0.4) (layer "B.Cu") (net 8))
 (segment (start 65.92 55.6) (end 64.2647 53.9447) (width 0.4) (layer "B.Cu") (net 8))
 (segment (start 80.54 56.9025) (end 80.54 57) (width 0.4) (layer "B.Cu") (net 8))
 (segment (start 53.92 55.6) (end 52.2149 57.3051) (width 0.4) (layer "B.Cu") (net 8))
 (segment (start 54.0827 75.5) (end 56 75.5) (width 0.4) (layer "B.Cu") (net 8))
 (segment (start 88.5 57) (end 86.7384 55.2384) (width 0.4) (layer "B.Cu") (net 8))
 (segment (start 84.2944 55.2384) (end 84.2944 52.0751) (width 0.4) (layer "B.Cu") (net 8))
 (segment (start 84.2944 52.0751) (end 83.6176 51.3983) (width 0.4) (layer "B.Cu") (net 8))
 (segment (start 70.1217 51.3983) (end 79.3383 51.3983) (width 0.4) (layer "B.Cu") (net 8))
 (segment (start 52.2149 65.8447) (end 51.6632 66.3964) (width 0.4) (layer "B.Cu") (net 8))
 (segment (start 79.3383 51.3983) (end 80.54 52.6) (width 0.4) (layer "B.Cu") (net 8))
 (segment (start 83.6176 51.3983) (end 81.7417 51.3983) (width 0.4) (layer "B.Cu") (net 8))
 (segment (start 84.2944 55.2384) (end 82.2041 55.2384) (width 0.4) (layer "B.Cu") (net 8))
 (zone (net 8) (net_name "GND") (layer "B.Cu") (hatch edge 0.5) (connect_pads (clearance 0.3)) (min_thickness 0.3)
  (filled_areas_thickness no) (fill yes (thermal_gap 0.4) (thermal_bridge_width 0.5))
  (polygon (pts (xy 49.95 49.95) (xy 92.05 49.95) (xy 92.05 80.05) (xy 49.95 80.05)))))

